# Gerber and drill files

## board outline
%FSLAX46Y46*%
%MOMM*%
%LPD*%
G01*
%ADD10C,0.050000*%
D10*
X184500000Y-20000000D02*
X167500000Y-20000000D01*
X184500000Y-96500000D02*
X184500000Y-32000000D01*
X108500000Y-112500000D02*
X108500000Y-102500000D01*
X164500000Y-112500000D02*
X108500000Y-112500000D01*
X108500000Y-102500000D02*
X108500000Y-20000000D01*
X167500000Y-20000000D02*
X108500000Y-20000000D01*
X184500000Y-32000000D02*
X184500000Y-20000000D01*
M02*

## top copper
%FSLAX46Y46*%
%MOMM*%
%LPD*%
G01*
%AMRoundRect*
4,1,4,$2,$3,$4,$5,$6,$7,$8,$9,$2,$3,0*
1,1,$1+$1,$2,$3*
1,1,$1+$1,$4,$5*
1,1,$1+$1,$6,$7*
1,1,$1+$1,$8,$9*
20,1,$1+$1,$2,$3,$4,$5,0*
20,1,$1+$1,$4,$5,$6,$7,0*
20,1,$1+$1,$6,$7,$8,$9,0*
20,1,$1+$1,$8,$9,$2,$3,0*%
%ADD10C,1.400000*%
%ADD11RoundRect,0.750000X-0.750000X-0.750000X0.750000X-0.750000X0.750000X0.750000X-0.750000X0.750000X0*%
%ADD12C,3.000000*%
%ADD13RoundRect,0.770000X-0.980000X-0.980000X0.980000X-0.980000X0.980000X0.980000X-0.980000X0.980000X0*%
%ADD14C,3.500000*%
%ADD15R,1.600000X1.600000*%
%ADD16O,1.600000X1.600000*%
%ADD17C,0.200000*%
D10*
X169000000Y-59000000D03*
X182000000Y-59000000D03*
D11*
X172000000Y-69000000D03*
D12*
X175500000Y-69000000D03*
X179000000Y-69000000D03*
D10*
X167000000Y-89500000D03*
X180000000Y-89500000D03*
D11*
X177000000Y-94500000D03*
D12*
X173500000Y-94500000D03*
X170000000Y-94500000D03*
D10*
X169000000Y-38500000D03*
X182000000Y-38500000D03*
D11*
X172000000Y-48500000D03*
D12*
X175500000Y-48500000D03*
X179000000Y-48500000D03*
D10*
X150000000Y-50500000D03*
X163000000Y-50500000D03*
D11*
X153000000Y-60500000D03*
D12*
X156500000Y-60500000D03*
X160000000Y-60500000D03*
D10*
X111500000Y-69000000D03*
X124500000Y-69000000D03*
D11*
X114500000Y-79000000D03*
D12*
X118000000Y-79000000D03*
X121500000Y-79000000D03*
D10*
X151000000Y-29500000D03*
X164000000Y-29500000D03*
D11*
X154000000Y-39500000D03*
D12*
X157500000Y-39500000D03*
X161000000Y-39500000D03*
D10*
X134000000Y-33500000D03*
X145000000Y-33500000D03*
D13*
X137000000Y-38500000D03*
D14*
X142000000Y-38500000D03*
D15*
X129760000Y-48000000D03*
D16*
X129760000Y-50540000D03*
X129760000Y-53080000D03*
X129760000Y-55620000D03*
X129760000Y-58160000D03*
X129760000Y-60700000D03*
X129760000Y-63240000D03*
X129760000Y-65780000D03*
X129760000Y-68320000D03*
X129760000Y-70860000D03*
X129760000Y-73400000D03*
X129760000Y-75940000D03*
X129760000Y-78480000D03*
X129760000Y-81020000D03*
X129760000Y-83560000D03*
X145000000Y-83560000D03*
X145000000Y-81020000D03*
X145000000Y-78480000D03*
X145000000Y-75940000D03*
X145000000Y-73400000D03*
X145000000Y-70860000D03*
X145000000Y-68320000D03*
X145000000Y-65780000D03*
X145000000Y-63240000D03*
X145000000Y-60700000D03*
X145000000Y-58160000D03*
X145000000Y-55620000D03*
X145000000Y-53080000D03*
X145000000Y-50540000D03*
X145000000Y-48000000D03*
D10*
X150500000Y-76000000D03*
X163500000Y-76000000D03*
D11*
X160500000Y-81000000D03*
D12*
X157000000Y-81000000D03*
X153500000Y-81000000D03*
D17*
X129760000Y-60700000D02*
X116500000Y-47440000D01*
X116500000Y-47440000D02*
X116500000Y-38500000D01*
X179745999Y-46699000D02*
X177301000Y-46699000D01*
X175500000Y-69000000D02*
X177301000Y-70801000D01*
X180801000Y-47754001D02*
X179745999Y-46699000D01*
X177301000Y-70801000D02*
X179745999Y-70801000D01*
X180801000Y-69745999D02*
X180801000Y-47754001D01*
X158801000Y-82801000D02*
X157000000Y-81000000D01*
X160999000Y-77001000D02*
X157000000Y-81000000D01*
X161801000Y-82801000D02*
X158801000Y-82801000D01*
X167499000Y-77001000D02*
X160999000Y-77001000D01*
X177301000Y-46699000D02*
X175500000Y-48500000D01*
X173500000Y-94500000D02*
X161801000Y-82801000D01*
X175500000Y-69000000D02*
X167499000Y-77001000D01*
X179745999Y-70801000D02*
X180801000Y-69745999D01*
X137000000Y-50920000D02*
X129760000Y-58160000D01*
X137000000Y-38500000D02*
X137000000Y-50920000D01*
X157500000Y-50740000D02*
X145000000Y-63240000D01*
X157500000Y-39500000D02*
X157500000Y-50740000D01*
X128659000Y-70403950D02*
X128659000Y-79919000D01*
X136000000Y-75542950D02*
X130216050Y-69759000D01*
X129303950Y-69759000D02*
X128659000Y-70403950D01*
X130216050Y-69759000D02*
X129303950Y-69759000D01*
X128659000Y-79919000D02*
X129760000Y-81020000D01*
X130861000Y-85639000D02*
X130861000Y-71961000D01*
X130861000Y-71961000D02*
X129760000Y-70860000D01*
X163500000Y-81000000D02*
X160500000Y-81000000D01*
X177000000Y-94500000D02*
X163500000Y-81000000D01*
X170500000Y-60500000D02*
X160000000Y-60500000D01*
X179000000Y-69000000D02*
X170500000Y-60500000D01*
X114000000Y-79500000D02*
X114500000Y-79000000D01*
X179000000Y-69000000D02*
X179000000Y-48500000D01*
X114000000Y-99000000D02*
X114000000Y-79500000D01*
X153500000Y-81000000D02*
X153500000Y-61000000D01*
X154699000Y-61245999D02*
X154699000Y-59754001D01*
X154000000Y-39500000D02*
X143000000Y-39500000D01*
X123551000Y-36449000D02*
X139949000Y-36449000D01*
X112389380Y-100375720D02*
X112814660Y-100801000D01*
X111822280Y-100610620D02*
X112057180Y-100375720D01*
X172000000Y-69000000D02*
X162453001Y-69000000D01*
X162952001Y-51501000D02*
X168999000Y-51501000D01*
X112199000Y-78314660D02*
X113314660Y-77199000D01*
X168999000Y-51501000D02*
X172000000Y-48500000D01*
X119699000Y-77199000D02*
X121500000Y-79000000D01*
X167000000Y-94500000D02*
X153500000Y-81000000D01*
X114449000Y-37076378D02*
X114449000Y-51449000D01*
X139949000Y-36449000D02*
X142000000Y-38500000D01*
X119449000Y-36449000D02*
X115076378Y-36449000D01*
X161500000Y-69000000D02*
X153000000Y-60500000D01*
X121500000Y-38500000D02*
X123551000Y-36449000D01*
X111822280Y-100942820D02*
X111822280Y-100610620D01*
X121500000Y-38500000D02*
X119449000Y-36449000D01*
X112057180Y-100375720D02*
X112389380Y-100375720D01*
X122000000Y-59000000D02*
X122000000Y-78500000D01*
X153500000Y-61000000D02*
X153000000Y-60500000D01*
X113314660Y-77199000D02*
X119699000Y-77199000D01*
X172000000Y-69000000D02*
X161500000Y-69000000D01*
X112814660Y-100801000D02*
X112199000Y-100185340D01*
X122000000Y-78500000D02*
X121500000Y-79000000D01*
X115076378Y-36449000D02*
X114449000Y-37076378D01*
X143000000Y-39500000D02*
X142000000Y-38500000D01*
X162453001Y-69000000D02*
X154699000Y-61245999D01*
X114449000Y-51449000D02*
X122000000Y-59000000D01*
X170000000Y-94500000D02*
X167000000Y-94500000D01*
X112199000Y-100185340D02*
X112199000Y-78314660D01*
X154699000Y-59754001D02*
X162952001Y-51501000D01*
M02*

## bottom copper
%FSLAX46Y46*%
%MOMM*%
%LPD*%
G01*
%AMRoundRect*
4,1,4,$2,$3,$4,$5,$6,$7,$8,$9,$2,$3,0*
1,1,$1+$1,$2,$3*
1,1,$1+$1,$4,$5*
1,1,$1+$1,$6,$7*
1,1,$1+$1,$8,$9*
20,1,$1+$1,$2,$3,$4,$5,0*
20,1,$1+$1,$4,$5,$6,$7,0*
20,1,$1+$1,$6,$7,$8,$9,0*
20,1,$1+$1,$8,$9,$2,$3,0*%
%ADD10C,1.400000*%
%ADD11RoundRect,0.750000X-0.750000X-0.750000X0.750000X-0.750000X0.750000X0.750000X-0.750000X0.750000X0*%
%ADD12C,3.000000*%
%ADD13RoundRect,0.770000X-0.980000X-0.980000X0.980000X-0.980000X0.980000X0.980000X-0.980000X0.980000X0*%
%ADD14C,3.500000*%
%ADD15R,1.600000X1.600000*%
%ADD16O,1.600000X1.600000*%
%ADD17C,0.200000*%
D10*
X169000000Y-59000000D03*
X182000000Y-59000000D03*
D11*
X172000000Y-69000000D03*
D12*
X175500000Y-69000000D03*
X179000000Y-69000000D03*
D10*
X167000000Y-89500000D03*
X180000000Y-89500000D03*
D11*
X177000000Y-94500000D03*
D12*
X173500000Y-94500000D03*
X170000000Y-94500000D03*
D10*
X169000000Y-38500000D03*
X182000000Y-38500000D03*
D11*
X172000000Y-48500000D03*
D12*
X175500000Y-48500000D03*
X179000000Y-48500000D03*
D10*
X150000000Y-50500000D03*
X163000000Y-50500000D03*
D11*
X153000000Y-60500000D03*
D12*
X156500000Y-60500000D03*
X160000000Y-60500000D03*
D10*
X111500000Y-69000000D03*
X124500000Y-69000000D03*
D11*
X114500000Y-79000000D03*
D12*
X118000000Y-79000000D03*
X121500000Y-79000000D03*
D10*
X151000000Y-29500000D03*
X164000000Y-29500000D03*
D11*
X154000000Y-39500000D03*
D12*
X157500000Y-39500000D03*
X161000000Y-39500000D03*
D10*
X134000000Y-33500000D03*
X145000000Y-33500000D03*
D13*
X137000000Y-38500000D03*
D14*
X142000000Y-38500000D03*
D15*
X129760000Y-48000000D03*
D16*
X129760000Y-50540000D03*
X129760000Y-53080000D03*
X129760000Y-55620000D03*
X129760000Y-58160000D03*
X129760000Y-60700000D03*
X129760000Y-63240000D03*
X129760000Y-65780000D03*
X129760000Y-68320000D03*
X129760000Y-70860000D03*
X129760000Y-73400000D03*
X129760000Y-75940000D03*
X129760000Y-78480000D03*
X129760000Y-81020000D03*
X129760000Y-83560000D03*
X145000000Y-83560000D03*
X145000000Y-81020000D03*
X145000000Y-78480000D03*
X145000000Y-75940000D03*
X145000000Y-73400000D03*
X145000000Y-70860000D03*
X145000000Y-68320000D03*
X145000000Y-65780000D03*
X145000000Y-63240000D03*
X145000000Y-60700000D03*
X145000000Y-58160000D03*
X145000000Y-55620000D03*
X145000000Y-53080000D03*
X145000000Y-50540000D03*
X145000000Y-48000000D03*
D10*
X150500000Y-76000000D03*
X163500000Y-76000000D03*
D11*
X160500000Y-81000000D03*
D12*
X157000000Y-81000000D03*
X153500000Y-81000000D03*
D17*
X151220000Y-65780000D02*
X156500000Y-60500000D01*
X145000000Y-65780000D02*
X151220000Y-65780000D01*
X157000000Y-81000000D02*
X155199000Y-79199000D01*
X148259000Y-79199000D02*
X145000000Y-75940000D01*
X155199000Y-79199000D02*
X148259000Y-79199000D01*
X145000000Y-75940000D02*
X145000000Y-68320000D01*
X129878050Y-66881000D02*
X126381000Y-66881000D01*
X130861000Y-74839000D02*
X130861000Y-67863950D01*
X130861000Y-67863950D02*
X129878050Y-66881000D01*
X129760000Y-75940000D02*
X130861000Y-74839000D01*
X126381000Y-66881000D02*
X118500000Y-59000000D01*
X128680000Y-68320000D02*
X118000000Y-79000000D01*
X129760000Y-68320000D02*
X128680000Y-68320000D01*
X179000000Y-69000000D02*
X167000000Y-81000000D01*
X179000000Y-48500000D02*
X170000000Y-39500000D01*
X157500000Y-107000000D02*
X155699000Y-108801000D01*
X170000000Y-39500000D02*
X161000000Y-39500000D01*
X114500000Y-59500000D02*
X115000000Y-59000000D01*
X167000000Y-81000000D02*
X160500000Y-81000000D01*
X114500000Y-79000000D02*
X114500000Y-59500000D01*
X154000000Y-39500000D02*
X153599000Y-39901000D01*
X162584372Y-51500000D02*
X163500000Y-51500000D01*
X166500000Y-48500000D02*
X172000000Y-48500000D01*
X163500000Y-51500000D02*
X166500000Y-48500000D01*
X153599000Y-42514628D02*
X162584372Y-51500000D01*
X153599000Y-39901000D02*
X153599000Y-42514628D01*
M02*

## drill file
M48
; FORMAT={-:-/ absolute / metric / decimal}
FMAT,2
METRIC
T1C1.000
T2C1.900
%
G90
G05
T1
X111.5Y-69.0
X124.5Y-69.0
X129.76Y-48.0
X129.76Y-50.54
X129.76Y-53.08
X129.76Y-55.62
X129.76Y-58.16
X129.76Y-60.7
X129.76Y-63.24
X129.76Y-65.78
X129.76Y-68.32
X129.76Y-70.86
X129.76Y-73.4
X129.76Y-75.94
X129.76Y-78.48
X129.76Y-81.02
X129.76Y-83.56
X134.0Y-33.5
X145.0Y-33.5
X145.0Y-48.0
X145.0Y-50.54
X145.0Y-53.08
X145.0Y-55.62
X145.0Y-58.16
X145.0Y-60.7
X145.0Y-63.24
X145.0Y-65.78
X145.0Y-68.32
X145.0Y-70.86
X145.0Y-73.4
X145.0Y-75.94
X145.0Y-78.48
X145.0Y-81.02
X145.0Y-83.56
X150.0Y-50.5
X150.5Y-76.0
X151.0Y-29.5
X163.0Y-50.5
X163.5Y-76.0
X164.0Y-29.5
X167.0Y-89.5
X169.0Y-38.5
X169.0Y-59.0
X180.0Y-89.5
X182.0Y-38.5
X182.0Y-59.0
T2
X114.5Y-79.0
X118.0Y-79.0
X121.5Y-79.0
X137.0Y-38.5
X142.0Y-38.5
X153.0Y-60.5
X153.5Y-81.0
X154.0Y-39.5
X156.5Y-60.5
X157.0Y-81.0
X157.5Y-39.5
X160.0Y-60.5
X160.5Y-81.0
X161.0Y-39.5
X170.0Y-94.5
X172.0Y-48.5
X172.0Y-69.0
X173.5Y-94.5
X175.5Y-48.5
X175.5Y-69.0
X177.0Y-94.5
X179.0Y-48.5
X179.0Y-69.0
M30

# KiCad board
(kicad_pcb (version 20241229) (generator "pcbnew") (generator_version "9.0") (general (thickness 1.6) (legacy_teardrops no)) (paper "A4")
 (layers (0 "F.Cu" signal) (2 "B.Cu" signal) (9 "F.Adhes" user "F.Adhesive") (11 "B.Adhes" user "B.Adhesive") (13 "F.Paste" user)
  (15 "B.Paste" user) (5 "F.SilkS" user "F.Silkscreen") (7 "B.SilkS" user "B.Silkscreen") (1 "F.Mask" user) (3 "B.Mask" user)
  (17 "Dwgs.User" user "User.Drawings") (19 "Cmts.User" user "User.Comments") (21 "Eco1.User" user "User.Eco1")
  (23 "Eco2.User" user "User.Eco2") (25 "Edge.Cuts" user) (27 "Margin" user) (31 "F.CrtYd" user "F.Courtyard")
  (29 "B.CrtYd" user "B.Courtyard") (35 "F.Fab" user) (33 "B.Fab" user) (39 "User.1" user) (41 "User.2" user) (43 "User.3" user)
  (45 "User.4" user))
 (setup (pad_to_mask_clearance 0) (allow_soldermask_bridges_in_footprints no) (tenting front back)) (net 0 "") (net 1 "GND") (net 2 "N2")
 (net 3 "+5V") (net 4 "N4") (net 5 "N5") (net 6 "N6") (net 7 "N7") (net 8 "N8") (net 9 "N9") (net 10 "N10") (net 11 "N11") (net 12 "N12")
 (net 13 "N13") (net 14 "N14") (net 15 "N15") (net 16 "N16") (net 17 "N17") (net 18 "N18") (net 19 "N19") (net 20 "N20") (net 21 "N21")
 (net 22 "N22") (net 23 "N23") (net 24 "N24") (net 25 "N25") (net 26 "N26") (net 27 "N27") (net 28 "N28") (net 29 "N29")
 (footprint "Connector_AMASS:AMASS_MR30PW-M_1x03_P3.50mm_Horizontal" (layer "F.Cu") (at 172 69)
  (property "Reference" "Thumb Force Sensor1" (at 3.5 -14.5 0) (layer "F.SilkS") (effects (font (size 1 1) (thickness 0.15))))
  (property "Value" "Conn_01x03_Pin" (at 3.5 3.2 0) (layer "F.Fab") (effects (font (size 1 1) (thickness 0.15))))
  (pad "" thru_hole circle (at -3 -10) (size 1.4 1.4) (drill 1) (layers "*.Cu" "*.Mask") (remove_unused_layers no))
  (pad "" thru_hole circle (at 10 -10) (size 1.4 1.4) (drill 1) (layers "*.Cu" "*.Mask") (remove_unused_layers no))
  (pad "1" thru_hole roundrect (at 0 0) (size 3 3) (drill 1.9) (layers "*.Cu" "*.Mask") (remove_unused_layers no) (roundrect_rratio 0.25)
   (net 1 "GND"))
  (pad "2" thru_hole circle (at 3.5 0) (size 3 3) (drill 1.9) (layers "*.Cu" "*.Mask") (remove_unused_layers no) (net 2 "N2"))
  (pad "3" thru_hole circle (at 7 0) (size 3 3) (drill 1.9) (layers "*.Cu" "*.Mask") (remove_unused_layers no) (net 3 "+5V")))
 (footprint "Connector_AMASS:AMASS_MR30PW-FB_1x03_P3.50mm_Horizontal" (layer "F.Cu") (at 177 94.5)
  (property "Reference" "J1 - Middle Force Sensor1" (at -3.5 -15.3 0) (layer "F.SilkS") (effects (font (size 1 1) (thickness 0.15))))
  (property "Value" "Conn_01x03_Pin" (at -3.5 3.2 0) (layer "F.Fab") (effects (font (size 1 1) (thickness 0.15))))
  (pad "" thru_hole circle (at -10 -5) (size 1.4 1.4) (drill 1) (layers "*.Cu" "*.Mask") (remove_unused_layers no))
  (pad "" thru_hole circle (at 3 -5 90) (size 1.4 1.4) (drill 1) (layers "*.Cu" "*.Mask") (remove_unused_layers no))
  (pad "1" thru_hole roundrect (at 0 0) (size 3 3) (drill 1.9) (layers "*.Cu" "*.Mask") (remove_unused_layers no) (roundrect_rratio 0.25)
   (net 3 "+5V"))
  (pad "2" thru_hole circle (at -3.5 0) (size 3 3) (drill 1.9) (layers "*.Cu" "*.Mask") (remove_unused_layers no) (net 2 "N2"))
  (pad "3" thru_hole circle (at -7 0) (size 3 3) (drill 1.9) (layers "*.Cu" "*.Mask") (remove_unused_layers no) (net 1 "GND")))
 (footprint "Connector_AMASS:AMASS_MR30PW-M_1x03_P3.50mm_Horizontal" (layer "F.Cu") (at 172 48.5)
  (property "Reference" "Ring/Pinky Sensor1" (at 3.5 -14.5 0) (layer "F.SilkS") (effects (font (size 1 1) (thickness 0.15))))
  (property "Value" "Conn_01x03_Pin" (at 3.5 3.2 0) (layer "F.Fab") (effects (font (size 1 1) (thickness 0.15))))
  (pad "" thru_hole circle (at -3 -10) (size 1.4 1.4) (drill 1) (layers "*.Cu" "*.Mask") (remove_unused_layers no))
  (pad "" thru_hole circle (at 10 -10) (size 1.4 1.4) (drill 1) (layers "*.Cu" "*.Mask") (remove_unused_layers no))
  (pad "1" thru_hole roundrect (at 0 0) (size 3 3) (drill 1.9) (layers "*.Cu" "*.Mask") (remove_unused_layers no) (roundrect_rratio 0.25)
   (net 1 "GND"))
  (pad "2" thru_hole circle (at 3.5 0) (size 3 3) (drill 1.9) (layers "*.Cu" "*.Mask") (remove_unused_layers no) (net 2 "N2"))
  (pad "3" thru_hole circle (at 7 0) (size 3 3) (drill 1.9) (layers "*.Cu" "*.Mask") (remove_unused_layers no) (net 3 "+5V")))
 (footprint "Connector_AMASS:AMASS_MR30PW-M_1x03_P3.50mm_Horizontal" (layer "F.Cu") (at 153 60.5)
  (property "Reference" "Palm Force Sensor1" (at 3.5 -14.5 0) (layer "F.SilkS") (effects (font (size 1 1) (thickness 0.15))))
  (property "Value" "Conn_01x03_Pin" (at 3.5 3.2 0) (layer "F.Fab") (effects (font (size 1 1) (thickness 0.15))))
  (pad "" thru_hole circle (at -3 -10) (size 1.4 1.4) (drill 1) (layers "*.Cu" "*.Mask") (remove_unused_layers no))
  (pad "" thru_hole circle (at 10 -10) (size 1.4 1.4) (drill 1) (layers "*.Cu" "*.Mask") (remove_unused_layers no))
  (pad "1" thru_hole roundrect (at 0 0) (size 3 3) (drill 1.9) (layers "*.Cu" "*.Mask") (remove_unused_layers no) (roundrect_rratio 0.25)
   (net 1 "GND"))
  (pad "2" thru_hole circle (at 3.5 0) (size 3 3) (drill 1.9) (layers "*.Cu" "*.Mask") (remove_unused_layers no) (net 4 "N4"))
  (pad "3" thru_hole circle (at 7 0) (size 3 3) (drill 1.9) (layers "*.Cu" "*.Mask") (remove_unused_layers no) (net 3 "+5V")))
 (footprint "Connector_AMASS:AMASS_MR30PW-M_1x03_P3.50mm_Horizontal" (layer "F.Cu") (at 114.5 79)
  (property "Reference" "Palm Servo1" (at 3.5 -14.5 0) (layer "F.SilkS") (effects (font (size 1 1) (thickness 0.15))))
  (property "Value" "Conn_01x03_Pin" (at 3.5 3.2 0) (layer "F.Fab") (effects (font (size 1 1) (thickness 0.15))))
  (pad "" thru_hole circle (at -3 -10) (size 1.4 1.4) (drill 1) (layers "*.Cu" "*.Mask") (remove_unused_layers no))
  (pad "" thru_hole circle (at 10 -10) (size 1.4 1.4) (drill 1) (layers "*.Cu" "*.Mask") (remove_unused_layers no))
  (pad "1" thru_hole roundrect (at 0 0) (size 3 3) (drill 1.9) (layers "*.Cu" "*.Mask") (remove_unused_layers no) (roundrect_rratio 0.25)
   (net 3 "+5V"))
  (pad "2" thru_hole circle (at 3.5 0) (size 3 3) (drill 1.9) (layers "*.Cu" "*.Mask") (remove_unused_layers no) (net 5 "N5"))
  (pad "3" thru_hole circle (at 7 0) (size 3 3) (drill 1.9) (layers "*.Cu" "*.Mask") (remove_unused_layers no) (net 1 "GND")))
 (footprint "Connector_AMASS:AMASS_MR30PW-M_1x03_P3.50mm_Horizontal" (layer "F.Cu") (at 154 39.5)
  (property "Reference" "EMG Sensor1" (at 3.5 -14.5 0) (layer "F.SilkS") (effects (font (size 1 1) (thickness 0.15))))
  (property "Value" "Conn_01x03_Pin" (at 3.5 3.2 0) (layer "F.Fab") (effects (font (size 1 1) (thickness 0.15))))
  (pad "" thru_hole circle (at -3 -10) (size 1.4 1.4) (drill 1) (layers "*.Cu" "*.Mask") (remove_unused_layers no))
  (pad "" thru_hole circle (at 10 -10) (size 1.4 1.4) (drill 1) (layers "*.Cu" "*.Mask") (remove_unused_layers no))
  (pad "1" thru_hole roundrect (at 0 0) (size 3 3) (drill 1.9) (layers "*.Cu" "*.Mask") (remove_unused_layers no) (roundrect_rratio 0.25)
   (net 1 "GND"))
  (pad "2" thru_hole circle (at 3.5 0) (size 3 3) (drill 1.9) (layers "*.Cu" "*.Mask") (remove_unused_layers no) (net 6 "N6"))
  (pad "3" thru_hole circle (at 7 0) (size 3 3) (drill 1.9) (layers "*.Cu" "*.Mask") (remove_unused_layers no) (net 3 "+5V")))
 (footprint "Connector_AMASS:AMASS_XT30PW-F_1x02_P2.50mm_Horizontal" (layer "F.Cu") (at 137 38.5)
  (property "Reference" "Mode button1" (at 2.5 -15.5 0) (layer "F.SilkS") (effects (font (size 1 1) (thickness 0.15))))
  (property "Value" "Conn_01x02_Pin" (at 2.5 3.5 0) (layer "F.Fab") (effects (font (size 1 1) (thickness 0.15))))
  (pad "" thru_hole circle (at -3 -5 90) (size 1.4 1.4) (drill 1) (layers "*.Cu" "*.Mask") (remove_unused_layers no))
  (pad "" thru_hole circle (at 8 -5) (size 1.4 1.4) (drill 1) (layers "*.Cu" "*.Mask") (remove_unused_layers no))
  (pad "1" thru_hole roundrect (at 0 0) (size 3.5 3.5) (drill 1.9) (layers "*.Cu" "*.Mask") (remove_unused_layers no)
   (roundrect_rratio 0.22) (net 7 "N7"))
  (pad "2" thru_hole circle (at 5 0) (size 3.5 3.5) (drill 1.9) (layers "*.Cu" "*.Mask") (remove_unused_layers no) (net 1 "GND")))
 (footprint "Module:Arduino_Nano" (layer "F.Cu") (at 129.76 48)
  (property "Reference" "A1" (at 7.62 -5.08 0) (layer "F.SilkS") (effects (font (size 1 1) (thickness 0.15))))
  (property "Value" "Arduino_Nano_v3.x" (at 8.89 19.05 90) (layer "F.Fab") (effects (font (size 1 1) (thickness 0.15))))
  (pad "1" thru_hole rect (at 0 0) (size 1.6 1.6) (drill 1) (layers "*.Cu" "*.Mask") (remove_unused_layers no) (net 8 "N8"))
  (pad "2" thru_hole oval (at 0 2.54) (size 1.6 1.6) (drill 1) (layers "*.Cu" "*.Mask") (remove_unused_layers no) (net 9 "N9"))
  (pad "3" thru_hole oval (at 0 5.08) (size 1.6 1.6) (drill 1) (layers "*.Cu" "*.Mask") (remove_unused_layers no) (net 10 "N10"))
  (pad "4" thru_hole oval (at 0 7.62) (size 1.6 1.6) (drill 1) (layers "*.Cu" "*.Mask") (remove_unused_layers no) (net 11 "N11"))
  (pad "5" thru_hole oval (at 0 10.16) (size 1.6 1.6) (drill 1) (layers "*.Cu" "*.Mask") (remove_unused_layers no) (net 7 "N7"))
  (pad "6" thru_hole oval (at 0 12.7) (size 1.6 1.6) (drill 1) (layers "*.Cu" "*.Mask") (remove_unused_layers no) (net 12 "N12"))
  (pad "7" thru_hole oval (at 0 15.24) (size 1.6 1.6) (drill 1) (layers "*.Cu" "*.Mask") (remove_unused_layers no) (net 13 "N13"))
  (pad "8" thru_hole oval (at 0 17.78) (size 1.6 1.6) (drill 1) (layers "*.Cu" "*.Mask") (remove_unused_layers no) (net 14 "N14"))
  (pad "9" thru_hole oval (at 0 20.32) (size 1.6 1.6) (drill 1) (layers "*.Cu" "*.Mask") (remove_unused_layers no) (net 5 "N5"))
  (pad "10" thru_hole oval (at 0 22.86) (size 1.6 1.6) (drill 1) (layers "*.Cu" "*.Mask") (remove_unused_layers no) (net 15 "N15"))
  (pad "11" thru_hole oval (at 0 25.4) (size 1.6 1.6) (drill 1) (layers "*.Cu" "*.Mask") (remove_unused_layers no) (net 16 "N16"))
  (pad "12" thru_hole oval (at 0 27.94) (size 1.6 1.6) (drill 1) (layers "*.Cu" "*.Mask") (remove_unused_layers no) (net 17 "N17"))
  (pad "13" thru_hole oval (at 0 30.48) (size 1.6 1.6) (drill 1) (layers "*.Cu" "*.Mask") (remove_unused_layers no) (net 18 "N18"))
  (pad "14" thru_hole oval (at 0 33.02) (size 1.6 1.6) (drill 1) (layers "*.Cu" "*.Mask") (remove_unused_layers no) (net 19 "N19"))
  (pad "15" thru_hole oval (at 0 35.56) (size 1.6 1.6) (drill 1) (layers "*.Cu" "*.Mask") (remove_unused_layers no) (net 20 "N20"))
  (pad "16" thru_hole oval (at 15.24 35.56) (size 1.6 1.6) (drill 1) (layers "*.Cu" "*.Mask") (remove_unused_layers no) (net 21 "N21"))
  (pad "17" thru_hole oval (at 15.24 33.02) (size 1.6 1.6) (drill 1) (layers "*.Cu" "*.Mask") (remove_unused_layers no) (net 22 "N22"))
  (pad "18" thru_hole oval (at 15.24 30.48) (size 1.6 1.6) (drill 1) (layers "*.Cu" "*.Mask") (remove_unused_layers no) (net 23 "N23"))
  (pad "19" thru_hole oval (at 15.24 27.94) (size 1.6 1.6) (drill 1) (layers "*.Cu" "*.Mask") (remove_unused_layers no) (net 2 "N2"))
  (pad "20" thru_hole oval (at 15.24 25.4) (size 1.6 1.6) (drill 1) (layers "*.Cu" "*.Mask") (remove_unused_layers no) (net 2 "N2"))
  (pad "21" thru_hole oval (at 15.24 22.86) (size 1.6 1.6) (drill 1) (layers "*.Cu" "*.Mask") (remove_unused_layers no) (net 2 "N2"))
  (pad "22" thru_hole oval (at 15.24 20.32) (size 1.6 1.6) (drill 1) (layers "*.Cu" "*.Mask") (remove_unused_layers no) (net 2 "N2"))
  (pad "23" thru_hole oval (at 15.24 17.78) (size 1.6 1.6) (drill 1) (layers "*.Cu" "*.Mask") (remove_unused_layers no) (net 4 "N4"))
  (pad "24" thru_hole oval (at 15.24 15.24) (size 1.6 1.6) (drill 1) (layers "*.Cu" "*.Mask") (remove_unused_layers no) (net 6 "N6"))
  (pad "25" thru_hole oval (at 15.24 12.7) (size 1.6 1.6) (drill 1) (layers "*.Cu" "*.Mask") (remove_unused_layers no) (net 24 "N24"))
  (pad "26" thru_hole oval (at 15.24 10.16) (size 1.6 1.6) (drill 1) (layers "*.Cu" "*.Mask") (remove_unused_layers no) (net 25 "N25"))
  (pad "27" thru_hole oval (at 15.24 7.62) (size 1.6 1.6) (drill 1) (layers "*.Cu" "*.Mask") (remove_unused_layers no) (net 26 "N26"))
  (pad "28" thru_hole oval (at 15.24 5.08) (size 1.6 1.6) (drill 1) (layers "*.Cu" "*.Mask") (remove_unused_layers no) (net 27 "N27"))
  (pad "29" thru_hole oval (at 15.24 2.54) (size 1.6 1.6) (drill 1) (layers "*.Cu" "*.Mask") (remove_unused_layers no) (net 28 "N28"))
  (pad "30" thru_hole oval (at 15.24 0) (size 1.6 1.6) (drill 1) (layers "*.Cu" "*.Mask") (remove_unused_layers no) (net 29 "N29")))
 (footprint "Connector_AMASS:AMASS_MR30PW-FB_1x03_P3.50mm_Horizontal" (layer "F.Cu") (at 160.5 81)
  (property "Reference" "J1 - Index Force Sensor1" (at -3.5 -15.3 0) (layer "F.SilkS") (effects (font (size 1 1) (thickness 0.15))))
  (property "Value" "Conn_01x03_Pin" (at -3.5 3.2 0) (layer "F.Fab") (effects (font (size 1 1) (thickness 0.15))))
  (pad "" thru_hole circle (at -10 -5) (size 1.4 1.4) (drill 1) (layers "*.Cu" "*.Mask") (remove_unused_layers no))
  (pad "" thru_hole circle (at 3 -5 90) (size 1.4 1.4) (drill 1) (layers "*.Cu" "*.Mask") (remove_unused_layers no))
  (pad "1" thru_hole roundrect (at 0 0) (size 3 3) (drill 1.9) (layers "*.Cu" "*.Mask") (remove_unused_layers no) (roundrect_rratio 0.25)
   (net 3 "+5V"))
  (pad "2" thru_hole circle (at -3.5 0) (size 3 3) (drill 1.9) (layers "*.Cu" "*.Mask") (remove_unused_layers no) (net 2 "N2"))
  (pad "3" thru_hole circle (at -7 0) (size 3 3) (drill 1.9) (layers "*.Cu" "*.Mask") (remove_unused_layers no) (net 1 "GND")))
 (gr_line (start 184.5 20) (end 167.5 20) (stroke (width 0.05) (type default)) (layer "Edge.Cuts"))
 (gr_line (start 184.5 96.5) (end 184.5 32) (stroke (width 0.05) (type default)) (layer "Edge.Cuts"))
 (gr_line (start 108.5 112.5) (end 108.5 102.5) (stroke (width 0.05) (type default)) (layer "Edge.Cuts"))
 (gr_line (start 164.5 112.5) (end 108.5 112.5) (stroke (width 0.05) (type default)) (layer "Edge.Cuts"))
 (gr_line (start 108.5 102.5) (end 108.5 20) (stroke (width 0.05) (type default)) (layer "Edge.Cuts"))
 (gr_line (start 167.5 20) (end 108.5 20) (stroke (width 0.05) (type default)) (layer "Edge.Cuts"))
 (gr_line (start 184.5 32) (end 184.5 20) (stroke (width 0.05) (type default)) (layer "Edge.Cuts"))
 (segment (start 129.76 60.7) (end 116.5 47.44) (width 0.2) (layer "F.Cu") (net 12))
 (segment (start 116.5 47.44) (end 116.5 38.5) (width 0.2) (layer "F.Cu") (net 12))
 (segment (start 151.22 65.78) (end 156.5 60.5) (width 0.2) (layer "B.Cu") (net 4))
 (segment (start 145 65.78) (end 151.22 65.78) (width 0.2) (layer "B.Cu") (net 4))
 (segment (start 179.745999 46.699) (end 177.301 46.699) (width 0.2) (layer "F.Cu") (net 2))
 (segment (start 175.5 69) (end 177.301 70.801) (width 0.2) (layer "F.Cu") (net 2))
 (segment (start 180.801 47.754001) (end 179.745999 46.699) (width 0.2) (layer "F.Cu") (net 2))
 (segment (start 177.301 70.801) (end 179.745999 70.801) (width 0.2) (layer "F.Cu") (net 2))
 (segment (start 180.801 69.745999) (end 180.801 47.754001) (width 0.2) (layer "F.Cu") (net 2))
 (segment (start 158.801 82.801) (end 157 81) (width 0.2) (layer "F.Cu") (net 2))
 (segment (start 160.999 77.001) (end 157 81) (width 0.2) (layer "F.Cu") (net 2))
 (segment (start 161.801 82.801) (end 158.801 82.801) (width 0.2) (layer "F.Cu") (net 2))
 (segment (start 167.499 77.001) (end 160.999 77.001) (width 0.2) (layer "F.Cu") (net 2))
 (segment (start 177.301 46.699) (end 175.5 48.5) (width 0.2) (layer "F.Cu") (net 2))
 (segment (start 173.5 94.5) (end 161.801 82.801) (width 0.2) (layer "F.Cu") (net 2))
 (segment (start 175.5 69) (end 167.499 77.001) (width 0.2) (layer "F.Cu") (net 2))
 (segment (start 179.745999 70.801) (end 180.801 69.745999) (width 0.2) (layer "F.Cu") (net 2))
 (segment (start 157 81) (end 155.199 79.199) (width 0.2) (layer "B.Cu") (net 2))
 (segment (start 148.259 79.199) (end 145 75.94) (width 0.2) (layer "B.Cu") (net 2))
 (segment (start 155.199 79.199) (end 148.259 79.199) (width 0.2) (layer "B.Cu") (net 2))
 (segment (start 145 75.94) (end 145 68.32) (width 0.2) (layer "B.Cu") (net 2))
 (segment (start 137 50.92) (end 129.76 58.16) (width 0.2) (layer "F.Cu") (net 7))
 (segment (start 137 38.5) (end 137 50.92) (width 0.2) (layer "F.Cu") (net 7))
 (segment (start 157.5 50.74) (end 145 63.24) (width 0.2) (layer "F.Cu") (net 6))
 (segment (start 157.5 39.5) (end 157.5 50.74) (width 0.2) (layer "F.Cu") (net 6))
 (segment (start 129.87805 66.881) (end 126.381 66.881) (width 0.2) (layer "B.Cu") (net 17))
 (segment (start 130.861 74.839) (end 130.861 67.86395) (width 0.2) (layer "B.Cu") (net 17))
 (segment (start 130.861 67.86395) (end 129.87805 66.881) (width 0.2) (layer "B.Cu") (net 17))
 (segment (start 129.76 75.94) (end 130.861 74.839) (width 0.2) (layer "B.Cu") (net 17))
 (segment (start 126.381 66.881) (end 118.5 59) (width 0.2) (layer "B.Cu") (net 17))
 (segment (start 128.659 70.40395) (end 128.659 79.919) (width 0.2) (layer "F.Cu") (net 19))
 (segment (start 136 75.54295) (end 130.21605 69.759) (width 0.2) (layer "F.Cu") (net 19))
 (segment (start 129.30395 69.759) (end 128.659 70.40395) (width 0.2) (layer "F.Cu") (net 19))
 (segment (start 130.21605 69.759) (end 129.30395 69.759) (width 0.2) (layer "F.Cu") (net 19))
 (segment (start 128.659 79.919) (end 129.76 81.02) (width 0.2) (layer "F.Cu") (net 19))
 (segment (start 130.861 85.639) (end 130.861 71.961) (width 0.2) (layer "F.Cu") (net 15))
 (segment (start 130.861 71.961) (end 129.76 70.86) (width 0.2) (layer "F.Cu") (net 15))
 (segment (start 128.68 68.32) (end 118 79) (width 0.2) (layer "B.Cu") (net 5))
 (segment (start 129.76 68.32) (end 128.68 68.32) (width 0.2) (layer "B.Cu") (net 5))
 (segment (start 163.5 81) (end 160.5 81) (width 0.2) (layer "F.Cu") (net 3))
 (segment (start 177 94.5) (end 163.5 81) (width 0.2) (layer "F.Cu") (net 3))
 (segment (start 170.5 60.5) (end 160 60.5) (width 0.2) (layer "F.Cu") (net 3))
 (segment (start 179 69) (end 170.5 60.5) (width 0.2) (layer "F.Cu") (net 3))
 (segment (start 114 79.5) (end 114.5 79) (width 0.2) (layer "F.Cu") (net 3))
 (segment (start 179 69) (end 179 48.5) (width 0.2) (layer "F.Cu") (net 3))
 (segment (start 114 99) (end 114 79.5) (width 0.2) (layer "F.Cu") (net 3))
 (segment (start 179 69) (end 167 81) (width 0.2) (layer "B.Cu") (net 3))
 (segment (start 179 48.5) (end 170 39.5) (width 0.2) (layer "B.Cu") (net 3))
 (segment (start 157.5 107) (end 155.699 108.801) (width 0.2) (layer "B.Cu") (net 3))
 (segment (start 170 39.5) (end 161 39.5) (width 0.2) (layer "B.Cu") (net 3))
 (segment (start 114.5 59.5) (end 115 59) (width 0.2) (layer "B.Cu") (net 3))
 (segment (start 167 81) (end 160.5 81) (width 0.2) (layer "B.Cu") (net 3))
 (segment (start 114.5 79) (end 114.5 59.5) (width 0.2) (layer "B.Cu") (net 3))
 (segment (start 153.5 81) (end 153.5 61) (width 0.2) (layer "F.Cu") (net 1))
 (segment (start 154.699 61.245999) (end 154.699 59.754001) (width 0.2) (layer "F.Cu") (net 1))
 (segment (start 154 39.5) (end 143 39.5) (width 0.2) (layer "F.Cu") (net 1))
 (segment (start 123.551 36.449) (end 139.949 36.449) (width 0.2) (layer "F.Cu") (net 1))
 (segment (start 112.38938 100.37572) (end 112.81466 100.801) (width 0.2) (layer "F.Cu") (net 1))
 (segment (start 111.82228 100.61062) (end 112.05718 100.37572) (width 0.2) (layer "F.Cu") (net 1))
 (segment (start 172 69) (end 162.453001 69) (width 0.2) (layer "F.Cu") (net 1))
 (segment (start 162.952001 51.501) (end 168.999 51.501) (width 0.2) (layer "F.Cu") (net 1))
 (segment (start 112.199 78.31466) (end 113.31466 77.199) (width 0.2) (layer "F.Cu") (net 1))
 (segment (start 168.999 51.501) (end 172 48.5) (width 0.2) (layer "F.Cu") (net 1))
 (segment (start 119.699 77.199) (end 121.5 79) (width 0.2) (layer "F.Cu") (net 1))
 (segment (start 167 94.5) (end 153.5 81) (width 0.2) (layer "F.Cu") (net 1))
 (segment (start 114.449 37.076378) (end 114.449 51.449) (width 0.2) (layer "F.Cu") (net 1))
 (segment (start 139.949 36.449) (end 142 38.5) (width 0.2) (layer "F.Cu") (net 1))
 (segment (start 119.449 36.449) (end 115.076378 36.449) (width 0.2) (layer "F.Cu") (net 1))
 (segment (start 161.5 69) (end 153 60.5) (width 0.2) (layer "F.Cu") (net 1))
 (segment (start 121.5 38.5) (end 123.551 36.449) (width 0.2) (layer "F.Cu") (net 1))
 (segment (start 111.82228 100.94282) (end 111.82228 100.61062) (width 0.2) (layer "F.Cu") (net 1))
 (segment (start 121.5 38.5) (end 119.449 36.449) (width 0.2) (layer "F.Cu") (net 1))
 (segment (start 112.05718 100.37572) (end 112.38938 100.37572) (width 0.2) (layer "F.Cu") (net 1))
 (segment (start 122 59) (end 122 78.5) (width 0.2) (layer "F.Cu") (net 1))
 (segment (start 153.5 61) (end 153 60.5) (width 0.2) (layer "F.Cu") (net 1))
 (segment (start 113.31466 77.199) (end 119.699 77.199) (width 0.2) (layer "F.Cu") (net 1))
 (segment (start 172 69) (end 161.5 69) (width 0.2) (layer "F.Cu") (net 1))
 (segment (start 112.81466 100.801) (end 112.199 100.18534) (width 0.2) (layer "F.Cu") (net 1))
 (segment (start 122 78.5) (end 121.5 79) (width 0.2) (layer "F.Cu") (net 1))
 (segment (start 115.076378 36.449) (end 114.449 37.076378) (width 0.2) (layer "F.Cu") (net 1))
 (segment (start 143 39.5) (end 142 38.5) (width 0.2) (layer "F.Cu") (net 1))
 (segment (start 162.453001 69) (end 154.699 61.245999) (width 0.2) (layer "F.Cu") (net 1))
 (segment (start 114.449 51.449) (end 122 59) (width 0.2) (layer "F.Cu") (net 1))
 (segment (start 170 94.5) (end 167 94.5) (width 0.2) (layer "F.Cu") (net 1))
 (segment (start 112.199 100.18534) (end 112.199 78.31466) (width 0.2) (layer "F.Cu") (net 1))
 (segment (start 154.699 59.754001) (end 162.952001 51.501) (width 0.2) (layer "F.Cu") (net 1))
 (segment (start 154 39.5) (end 153.599 39.901) (width 0.2) (layer "B.Cu") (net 1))
 (segment (start 162.584372 51.5) (end 163.5 51.5) (width 0.2) (layer "B.Cu") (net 1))
 (segment (start 166.5 48.5) (end 172 48.5) (width 0.2) (layer "B.Cu") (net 1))
 (segment (start 163.5 51.5) (end 166.5 48.5) (width 0.2) (layer "B.Cu") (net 1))
 (segment (start 153.599 42.514628) (end 162.584372 51.5) (width 0.2) (layer "B.Cu") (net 1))
 (segment (start 153.599 39.901) (end 153.599 42.514628) (width 0.2) (layer "B.Cu") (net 1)))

